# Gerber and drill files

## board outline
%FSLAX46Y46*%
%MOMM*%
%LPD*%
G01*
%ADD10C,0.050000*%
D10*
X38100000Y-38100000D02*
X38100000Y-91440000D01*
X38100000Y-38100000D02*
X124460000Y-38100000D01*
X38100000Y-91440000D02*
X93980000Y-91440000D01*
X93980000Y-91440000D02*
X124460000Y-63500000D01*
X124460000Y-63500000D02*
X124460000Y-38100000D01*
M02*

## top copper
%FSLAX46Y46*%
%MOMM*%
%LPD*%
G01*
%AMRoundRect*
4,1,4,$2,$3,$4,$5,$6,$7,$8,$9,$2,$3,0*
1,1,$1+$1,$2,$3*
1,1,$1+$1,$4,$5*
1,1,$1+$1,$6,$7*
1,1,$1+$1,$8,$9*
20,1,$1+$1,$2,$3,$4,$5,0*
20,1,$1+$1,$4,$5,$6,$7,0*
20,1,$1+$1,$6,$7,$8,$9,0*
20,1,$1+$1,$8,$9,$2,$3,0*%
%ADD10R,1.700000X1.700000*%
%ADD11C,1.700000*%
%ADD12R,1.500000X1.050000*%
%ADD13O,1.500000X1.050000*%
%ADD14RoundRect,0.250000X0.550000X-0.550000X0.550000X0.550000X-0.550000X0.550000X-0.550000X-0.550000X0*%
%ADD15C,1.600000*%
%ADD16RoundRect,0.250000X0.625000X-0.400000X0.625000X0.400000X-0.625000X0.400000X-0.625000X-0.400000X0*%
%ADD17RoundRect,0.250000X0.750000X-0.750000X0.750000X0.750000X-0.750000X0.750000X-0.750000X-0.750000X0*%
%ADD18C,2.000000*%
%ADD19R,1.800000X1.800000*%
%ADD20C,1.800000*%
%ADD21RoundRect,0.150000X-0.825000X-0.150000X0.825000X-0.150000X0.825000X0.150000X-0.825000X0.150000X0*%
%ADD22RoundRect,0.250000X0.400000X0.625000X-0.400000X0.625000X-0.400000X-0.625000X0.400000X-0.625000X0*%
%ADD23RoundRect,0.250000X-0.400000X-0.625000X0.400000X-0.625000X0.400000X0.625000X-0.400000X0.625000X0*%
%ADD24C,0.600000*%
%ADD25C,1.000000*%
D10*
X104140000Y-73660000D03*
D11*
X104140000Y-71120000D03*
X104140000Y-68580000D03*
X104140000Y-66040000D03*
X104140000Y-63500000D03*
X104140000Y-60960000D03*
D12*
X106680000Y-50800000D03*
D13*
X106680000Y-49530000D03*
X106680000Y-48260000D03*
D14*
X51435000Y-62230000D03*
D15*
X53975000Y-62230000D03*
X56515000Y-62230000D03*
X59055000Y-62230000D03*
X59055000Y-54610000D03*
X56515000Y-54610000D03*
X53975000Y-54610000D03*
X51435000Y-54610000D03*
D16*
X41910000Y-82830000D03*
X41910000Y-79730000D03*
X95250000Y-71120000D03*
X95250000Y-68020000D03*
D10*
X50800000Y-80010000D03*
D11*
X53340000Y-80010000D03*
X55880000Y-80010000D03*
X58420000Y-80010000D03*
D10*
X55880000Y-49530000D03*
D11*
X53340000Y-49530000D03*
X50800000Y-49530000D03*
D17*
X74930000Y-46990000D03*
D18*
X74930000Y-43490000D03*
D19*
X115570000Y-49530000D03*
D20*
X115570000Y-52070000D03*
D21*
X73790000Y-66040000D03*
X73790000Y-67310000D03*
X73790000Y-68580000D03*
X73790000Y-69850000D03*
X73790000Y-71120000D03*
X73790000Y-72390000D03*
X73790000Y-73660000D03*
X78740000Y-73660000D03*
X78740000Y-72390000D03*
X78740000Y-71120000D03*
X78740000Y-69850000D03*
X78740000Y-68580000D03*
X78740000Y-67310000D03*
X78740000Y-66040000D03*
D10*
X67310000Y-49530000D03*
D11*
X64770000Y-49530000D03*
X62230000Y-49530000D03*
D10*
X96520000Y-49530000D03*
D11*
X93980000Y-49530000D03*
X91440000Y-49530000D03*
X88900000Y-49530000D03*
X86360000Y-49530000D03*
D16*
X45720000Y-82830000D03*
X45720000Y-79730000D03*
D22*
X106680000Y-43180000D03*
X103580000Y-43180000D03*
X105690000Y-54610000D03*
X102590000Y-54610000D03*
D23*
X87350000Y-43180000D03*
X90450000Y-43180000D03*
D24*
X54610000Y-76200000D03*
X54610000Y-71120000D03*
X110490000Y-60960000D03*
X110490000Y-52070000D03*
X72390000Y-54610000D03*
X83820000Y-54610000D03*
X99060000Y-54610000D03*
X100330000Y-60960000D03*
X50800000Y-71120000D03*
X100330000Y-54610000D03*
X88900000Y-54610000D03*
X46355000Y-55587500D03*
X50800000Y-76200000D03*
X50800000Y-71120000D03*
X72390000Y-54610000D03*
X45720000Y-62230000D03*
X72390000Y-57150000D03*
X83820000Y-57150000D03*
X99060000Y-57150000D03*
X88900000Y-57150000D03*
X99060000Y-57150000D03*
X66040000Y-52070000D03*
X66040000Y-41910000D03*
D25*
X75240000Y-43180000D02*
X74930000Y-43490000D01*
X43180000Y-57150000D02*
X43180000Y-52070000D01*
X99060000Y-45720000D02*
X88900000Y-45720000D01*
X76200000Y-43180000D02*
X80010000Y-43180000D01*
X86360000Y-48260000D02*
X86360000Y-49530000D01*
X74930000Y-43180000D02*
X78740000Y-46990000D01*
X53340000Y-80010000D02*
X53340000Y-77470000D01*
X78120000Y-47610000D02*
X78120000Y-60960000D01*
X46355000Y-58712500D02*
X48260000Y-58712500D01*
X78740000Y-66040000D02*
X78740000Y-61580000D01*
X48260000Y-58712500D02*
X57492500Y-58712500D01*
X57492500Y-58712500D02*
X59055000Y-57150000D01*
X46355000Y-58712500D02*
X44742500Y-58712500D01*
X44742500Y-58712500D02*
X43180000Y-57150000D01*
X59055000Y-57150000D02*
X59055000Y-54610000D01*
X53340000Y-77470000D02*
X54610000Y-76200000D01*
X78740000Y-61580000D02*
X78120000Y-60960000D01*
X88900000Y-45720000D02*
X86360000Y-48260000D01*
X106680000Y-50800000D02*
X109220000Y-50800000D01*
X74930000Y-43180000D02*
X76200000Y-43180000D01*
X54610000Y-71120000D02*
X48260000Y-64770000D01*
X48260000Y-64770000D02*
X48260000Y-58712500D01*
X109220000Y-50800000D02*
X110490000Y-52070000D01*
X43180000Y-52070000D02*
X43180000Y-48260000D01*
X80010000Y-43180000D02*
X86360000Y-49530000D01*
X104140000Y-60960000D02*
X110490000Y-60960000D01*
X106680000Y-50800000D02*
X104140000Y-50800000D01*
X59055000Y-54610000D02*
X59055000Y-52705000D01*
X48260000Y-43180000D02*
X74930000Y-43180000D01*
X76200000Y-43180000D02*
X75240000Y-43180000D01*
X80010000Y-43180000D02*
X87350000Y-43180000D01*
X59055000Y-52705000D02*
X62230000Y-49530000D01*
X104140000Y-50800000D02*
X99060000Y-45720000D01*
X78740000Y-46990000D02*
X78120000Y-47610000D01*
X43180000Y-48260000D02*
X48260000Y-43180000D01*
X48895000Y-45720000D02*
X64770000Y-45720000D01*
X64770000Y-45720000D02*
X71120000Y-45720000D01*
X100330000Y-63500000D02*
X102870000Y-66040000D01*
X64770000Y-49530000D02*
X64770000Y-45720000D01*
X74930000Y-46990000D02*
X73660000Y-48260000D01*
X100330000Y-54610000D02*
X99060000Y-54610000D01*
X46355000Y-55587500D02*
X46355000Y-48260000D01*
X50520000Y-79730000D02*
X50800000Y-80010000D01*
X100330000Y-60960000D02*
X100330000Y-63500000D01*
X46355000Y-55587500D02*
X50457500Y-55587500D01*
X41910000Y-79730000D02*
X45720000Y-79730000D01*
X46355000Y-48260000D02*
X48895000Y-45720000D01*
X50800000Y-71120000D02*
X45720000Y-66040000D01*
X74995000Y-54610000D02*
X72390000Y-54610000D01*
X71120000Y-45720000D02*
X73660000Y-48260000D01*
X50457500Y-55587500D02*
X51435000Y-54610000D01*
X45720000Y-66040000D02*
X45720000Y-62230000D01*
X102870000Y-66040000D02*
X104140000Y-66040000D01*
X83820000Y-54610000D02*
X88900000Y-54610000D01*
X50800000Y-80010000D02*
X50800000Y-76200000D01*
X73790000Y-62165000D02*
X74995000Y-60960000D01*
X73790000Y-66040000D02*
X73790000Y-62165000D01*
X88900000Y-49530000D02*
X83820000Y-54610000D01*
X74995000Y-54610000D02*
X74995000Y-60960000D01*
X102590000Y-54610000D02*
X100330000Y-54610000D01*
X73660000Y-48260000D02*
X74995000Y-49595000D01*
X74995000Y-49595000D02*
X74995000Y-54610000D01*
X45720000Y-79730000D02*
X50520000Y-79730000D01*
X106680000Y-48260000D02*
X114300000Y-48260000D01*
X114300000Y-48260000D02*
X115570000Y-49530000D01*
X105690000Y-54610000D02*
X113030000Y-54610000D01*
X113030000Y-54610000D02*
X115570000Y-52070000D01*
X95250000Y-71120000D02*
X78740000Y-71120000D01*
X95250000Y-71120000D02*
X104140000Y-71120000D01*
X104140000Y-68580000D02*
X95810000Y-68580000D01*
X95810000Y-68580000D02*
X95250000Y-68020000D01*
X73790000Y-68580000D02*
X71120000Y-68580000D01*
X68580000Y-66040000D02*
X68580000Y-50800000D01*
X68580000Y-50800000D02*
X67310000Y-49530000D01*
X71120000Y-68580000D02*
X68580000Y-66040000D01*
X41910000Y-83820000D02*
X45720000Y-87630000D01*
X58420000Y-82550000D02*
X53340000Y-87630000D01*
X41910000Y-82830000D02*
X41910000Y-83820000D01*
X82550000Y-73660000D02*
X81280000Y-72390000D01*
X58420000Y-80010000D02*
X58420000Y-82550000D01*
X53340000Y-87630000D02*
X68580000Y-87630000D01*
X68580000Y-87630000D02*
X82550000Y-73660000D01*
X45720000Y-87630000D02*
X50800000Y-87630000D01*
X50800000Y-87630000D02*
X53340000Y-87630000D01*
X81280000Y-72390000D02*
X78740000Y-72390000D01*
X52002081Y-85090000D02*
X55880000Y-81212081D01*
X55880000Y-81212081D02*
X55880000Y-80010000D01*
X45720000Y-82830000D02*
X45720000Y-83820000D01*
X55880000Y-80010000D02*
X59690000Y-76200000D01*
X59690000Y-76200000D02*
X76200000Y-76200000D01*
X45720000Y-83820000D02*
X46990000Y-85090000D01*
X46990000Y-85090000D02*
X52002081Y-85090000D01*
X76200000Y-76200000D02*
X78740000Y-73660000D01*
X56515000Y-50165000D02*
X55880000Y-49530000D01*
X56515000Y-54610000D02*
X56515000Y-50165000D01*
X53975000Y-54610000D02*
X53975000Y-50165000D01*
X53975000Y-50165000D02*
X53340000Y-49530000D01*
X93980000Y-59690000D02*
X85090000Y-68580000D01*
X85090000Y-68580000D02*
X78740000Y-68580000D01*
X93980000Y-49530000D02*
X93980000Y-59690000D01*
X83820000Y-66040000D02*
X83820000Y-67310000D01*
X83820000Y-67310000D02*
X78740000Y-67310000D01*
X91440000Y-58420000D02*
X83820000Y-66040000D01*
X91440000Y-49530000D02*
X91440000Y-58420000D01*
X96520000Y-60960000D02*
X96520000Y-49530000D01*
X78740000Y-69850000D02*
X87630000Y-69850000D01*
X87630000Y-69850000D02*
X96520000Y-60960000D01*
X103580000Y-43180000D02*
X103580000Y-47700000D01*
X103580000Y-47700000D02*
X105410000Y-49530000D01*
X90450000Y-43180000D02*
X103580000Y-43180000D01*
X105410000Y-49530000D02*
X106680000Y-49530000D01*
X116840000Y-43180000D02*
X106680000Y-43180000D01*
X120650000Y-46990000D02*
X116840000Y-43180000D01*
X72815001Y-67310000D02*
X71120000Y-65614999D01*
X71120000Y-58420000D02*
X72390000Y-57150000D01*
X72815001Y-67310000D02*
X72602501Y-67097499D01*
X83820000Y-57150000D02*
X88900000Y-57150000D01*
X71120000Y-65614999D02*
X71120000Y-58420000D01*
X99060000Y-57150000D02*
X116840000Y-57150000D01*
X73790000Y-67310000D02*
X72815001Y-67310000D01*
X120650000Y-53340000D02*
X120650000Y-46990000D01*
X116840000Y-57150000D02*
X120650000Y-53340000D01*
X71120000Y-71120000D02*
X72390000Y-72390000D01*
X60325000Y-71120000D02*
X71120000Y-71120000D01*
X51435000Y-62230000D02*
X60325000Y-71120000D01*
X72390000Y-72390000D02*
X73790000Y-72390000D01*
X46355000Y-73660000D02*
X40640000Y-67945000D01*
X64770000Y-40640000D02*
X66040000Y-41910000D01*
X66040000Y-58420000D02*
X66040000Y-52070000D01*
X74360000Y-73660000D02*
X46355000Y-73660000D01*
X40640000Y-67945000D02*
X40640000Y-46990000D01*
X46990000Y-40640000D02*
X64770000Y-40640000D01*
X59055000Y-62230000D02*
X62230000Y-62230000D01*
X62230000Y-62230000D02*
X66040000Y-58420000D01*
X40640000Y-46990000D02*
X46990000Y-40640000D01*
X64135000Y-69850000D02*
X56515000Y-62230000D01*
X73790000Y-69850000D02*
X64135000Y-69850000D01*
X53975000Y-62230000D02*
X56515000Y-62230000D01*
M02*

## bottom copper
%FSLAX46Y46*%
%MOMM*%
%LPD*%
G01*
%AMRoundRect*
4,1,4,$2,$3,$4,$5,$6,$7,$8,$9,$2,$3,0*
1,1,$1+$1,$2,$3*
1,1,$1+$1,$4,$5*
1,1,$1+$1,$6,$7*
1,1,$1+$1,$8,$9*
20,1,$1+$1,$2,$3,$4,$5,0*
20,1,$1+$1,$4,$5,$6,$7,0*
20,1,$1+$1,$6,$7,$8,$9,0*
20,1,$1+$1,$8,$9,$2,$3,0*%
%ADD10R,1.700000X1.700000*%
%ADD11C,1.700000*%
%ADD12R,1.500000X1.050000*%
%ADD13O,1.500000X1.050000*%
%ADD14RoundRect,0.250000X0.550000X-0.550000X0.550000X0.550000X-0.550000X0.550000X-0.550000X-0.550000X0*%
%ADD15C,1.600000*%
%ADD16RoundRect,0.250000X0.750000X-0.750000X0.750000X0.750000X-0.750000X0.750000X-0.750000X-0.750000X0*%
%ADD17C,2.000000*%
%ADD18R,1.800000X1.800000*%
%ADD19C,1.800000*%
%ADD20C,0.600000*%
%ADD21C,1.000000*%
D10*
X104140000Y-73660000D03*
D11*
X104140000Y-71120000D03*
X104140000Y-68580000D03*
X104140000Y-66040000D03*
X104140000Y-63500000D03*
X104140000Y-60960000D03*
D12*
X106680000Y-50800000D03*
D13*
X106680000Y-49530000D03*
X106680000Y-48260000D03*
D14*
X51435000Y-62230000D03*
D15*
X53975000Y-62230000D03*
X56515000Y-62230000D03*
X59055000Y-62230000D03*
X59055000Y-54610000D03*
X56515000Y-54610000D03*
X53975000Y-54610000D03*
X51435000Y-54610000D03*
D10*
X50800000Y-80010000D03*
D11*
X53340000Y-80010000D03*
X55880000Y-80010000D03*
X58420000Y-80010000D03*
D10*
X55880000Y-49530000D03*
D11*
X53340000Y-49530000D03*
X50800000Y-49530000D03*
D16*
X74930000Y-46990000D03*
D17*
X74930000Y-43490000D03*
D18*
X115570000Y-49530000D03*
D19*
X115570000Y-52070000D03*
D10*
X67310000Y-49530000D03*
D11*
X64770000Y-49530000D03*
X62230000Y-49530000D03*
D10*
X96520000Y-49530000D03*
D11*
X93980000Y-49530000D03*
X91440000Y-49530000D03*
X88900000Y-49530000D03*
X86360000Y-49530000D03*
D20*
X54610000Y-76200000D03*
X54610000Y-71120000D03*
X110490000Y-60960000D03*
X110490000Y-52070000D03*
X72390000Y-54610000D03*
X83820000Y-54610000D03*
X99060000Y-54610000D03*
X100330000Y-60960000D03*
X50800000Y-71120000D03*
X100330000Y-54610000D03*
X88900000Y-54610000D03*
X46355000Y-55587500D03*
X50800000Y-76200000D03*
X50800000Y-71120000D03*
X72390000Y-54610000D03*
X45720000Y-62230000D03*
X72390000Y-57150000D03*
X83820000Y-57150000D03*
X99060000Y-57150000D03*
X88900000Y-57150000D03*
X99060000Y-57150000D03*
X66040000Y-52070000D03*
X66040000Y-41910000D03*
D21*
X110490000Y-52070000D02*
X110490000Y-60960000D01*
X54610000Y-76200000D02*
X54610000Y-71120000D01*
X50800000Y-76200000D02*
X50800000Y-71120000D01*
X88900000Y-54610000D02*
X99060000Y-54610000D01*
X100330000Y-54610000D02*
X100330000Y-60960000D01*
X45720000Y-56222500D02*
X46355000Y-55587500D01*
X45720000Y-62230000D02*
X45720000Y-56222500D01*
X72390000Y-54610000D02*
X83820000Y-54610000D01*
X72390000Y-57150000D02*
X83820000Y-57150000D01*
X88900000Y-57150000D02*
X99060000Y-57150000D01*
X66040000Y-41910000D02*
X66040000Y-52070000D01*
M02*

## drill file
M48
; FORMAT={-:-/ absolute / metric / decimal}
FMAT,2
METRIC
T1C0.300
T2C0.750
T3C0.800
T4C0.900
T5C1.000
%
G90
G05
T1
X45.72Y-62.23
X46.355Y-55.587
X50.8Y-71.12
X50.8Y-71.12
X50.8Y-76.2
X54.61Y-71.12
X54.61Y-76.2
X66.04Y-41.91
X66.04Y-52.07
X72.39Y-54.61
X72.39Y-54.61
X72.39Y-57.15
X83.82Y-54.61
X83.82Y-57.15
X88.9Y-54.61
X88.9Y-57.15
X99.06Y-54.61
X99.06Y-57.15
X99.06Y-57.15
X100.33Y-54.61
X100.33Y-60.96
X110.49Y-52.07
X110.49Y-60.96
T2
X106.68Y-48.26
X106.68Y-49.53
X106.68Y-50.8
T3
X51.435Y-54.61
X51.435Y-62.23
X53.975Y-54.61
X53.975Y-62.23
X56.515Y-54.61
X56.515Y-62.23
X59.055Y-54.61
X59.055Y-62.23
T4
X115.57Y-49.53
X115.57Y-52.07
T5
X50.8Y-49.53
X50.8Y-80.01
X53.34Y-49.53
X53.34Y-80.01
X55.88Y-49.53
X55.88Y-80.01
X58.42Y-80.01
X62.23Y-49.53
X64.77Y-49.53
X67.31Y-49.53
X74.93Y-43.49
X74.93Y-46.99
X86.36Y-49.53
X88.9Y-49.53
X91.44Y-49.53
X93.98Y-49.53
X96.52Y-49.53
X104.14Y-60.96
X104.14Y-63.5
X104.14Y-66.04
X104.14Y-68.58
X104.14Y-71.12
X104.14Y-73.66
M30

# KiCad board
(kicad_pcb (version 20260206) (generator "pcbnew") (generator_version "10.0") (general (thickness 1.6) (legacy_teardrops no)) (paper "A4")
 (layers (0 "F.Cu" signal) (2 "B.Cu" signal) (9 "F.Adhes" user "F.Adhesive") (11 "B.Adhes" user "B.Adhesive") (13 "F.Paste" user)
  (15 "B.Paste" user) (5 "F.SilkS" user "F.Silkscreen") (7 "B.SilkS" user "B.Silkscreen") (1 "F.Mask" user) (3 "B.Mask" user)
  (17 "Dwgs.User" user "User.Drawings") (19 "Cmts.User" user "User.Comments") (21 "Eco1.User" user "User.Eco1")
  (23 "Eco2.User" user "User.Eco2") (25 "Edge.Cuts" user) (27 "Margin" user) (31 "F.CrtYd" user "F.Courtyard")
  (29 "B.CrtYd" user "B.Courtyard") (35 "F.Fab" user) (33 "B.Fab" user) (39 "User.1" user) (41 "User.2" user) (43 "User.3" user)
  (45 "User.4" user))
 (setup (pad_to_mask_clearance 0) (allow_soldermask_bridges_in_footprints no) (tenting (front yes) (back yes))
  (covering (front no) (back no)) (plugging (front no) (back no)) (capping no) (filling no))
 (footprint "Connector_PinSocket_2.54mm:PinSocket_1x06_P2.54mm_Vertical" (layer "F.Cu") (at 104.14 73.66 180)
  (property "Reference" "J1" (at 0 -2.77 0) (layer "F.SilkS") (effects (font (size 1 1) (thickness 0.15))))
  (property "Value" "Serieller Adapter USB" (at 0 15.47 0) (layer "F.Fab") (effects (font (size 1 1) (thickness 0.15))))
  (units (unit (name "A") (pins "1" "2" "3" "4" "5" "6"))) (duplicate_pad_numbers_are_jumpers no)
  (pad "1" thru_hole rect (at 0 0 180) (size 1.7 1.7) (drill 1) (layers "*.Cu" "*.Mask") (remove_unused_layers no)
   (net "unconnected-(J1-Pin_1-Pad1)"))
  (pad "2" thru_hole circle (at 0 2.54 180) (size 1.7 1.7) (drill 1) (layers "*.Cu" "*.Mask") (remove_unused_layers no)
   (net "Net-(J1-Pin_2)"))
  (pad "3" thru_hole circle (at 0 5.08 180) (size 1.7 1.7) (drill 1) (layers "*.Cu" "*.Mask") (remove_unused_layers no)
   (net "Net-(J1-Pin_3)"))
  (pad "4" thru_hole circle (at 0 7.62 180) (size 1.7 1.7) (drill 1) (layers "*.Cu" "*.Mask") (remove_unused_layers no) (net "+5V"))
  (pad "5" thru_hole circle (at 0 10.16 180) (size 1.7 1.7) (drill 1) (layers "*.Cu" "*.Mask") (remove_unused_layers no)
   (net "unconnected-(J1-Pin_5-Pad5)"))
  (pad "6" thru_hole circle (at 0 12.7 180) (size 1.7 1.7) (drill 1) (layers "*.Cu" "*.Mask") (remove_unused_layers no) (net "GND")))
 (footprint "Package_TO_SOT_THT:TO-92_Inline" (layer "F.Cu") (at 106.68 50.8 90)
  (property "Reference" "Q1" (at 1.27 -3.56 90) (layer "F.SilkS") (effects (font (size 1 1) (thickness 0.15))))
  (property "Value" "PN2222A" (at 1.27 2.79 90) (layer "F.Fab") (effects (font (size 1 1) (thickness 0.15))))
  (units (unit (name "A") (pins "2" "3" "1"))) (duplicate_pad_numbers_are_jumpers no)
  (pad "1" thru_hole rect (at 0 0 90) (size 1.05 1.5) (drill 0.75) (layers "*.Cu" "*.Mask") (remove_unused_layers no) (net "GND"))
  (pad "2" thru_hole oval (at 1.27 0 90) (size 1.05 1.5) (drill 0.75) (layers "*.Cu" "*.Mask") (remove_unused_layers no) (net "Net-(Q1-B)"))
  (pad "3" thru_hole oval (at 2.54 0 90) (size 1.05 1.5) (drill 0.75) (layers "*.Cu" "*.Mask") (remove_unused_layers no) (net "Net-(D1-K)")))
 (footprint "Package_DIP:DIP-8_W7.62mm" (layer "F.Cu") (at 51.435 62.23 90)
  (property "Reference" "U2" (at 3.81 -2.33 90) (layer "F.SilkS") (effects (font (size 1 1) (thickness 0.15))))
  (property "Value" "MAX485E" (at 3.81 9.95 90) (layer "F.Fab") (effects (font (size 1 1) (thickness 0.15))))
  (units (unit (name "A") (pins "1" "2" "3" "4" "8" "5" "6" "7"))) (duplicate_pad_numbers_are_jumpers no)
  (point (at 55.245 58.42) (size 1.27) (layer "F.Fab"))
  (pad "1" thru_hole roundrect (at 0 0 90) (size 1.6 1.6) (drill 0.8) (layers "*.Cu" "*.Mask") (remove_unused_layers no)
   (roundrect_rratio 0.15625) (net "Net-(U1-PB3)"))
  (pad "2" thru_hole circle (at 0 2.54 90) (size 1.6 1.6) (drill 0.8) (layers "*.Cu" "*.Mask") (remove_unused_layers no)
   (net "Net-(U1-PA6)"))
  (pad "3" thru_hole circle (at 0 5.08 90) (size 1.6 1.6) (drill 0.8) (layers "*.Cu" "*.Mask") (remove_unused_layers no)
   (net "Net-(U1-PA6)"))
  (pad "4" thru_hole circle (at 0 7.62 90) (size 1.6 1.6) (drill 0.8) (layers "*.Cu" "*.Mask") (remove_unused_layers no)
   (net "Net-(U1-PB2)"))
  (pad "5" thru_hole circle (at 7.62 7.62 90) (size 1.6 1.6) (drill 0.8) (layers "*.Cu" "*.Mask") (remove_unused_layers no) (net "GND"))
  (pad "6" thru_hole circle (at 7.62 5.08 90) (size 1.6 1.6) (drill 0.8) (layers "*.Cu" "*.Mask") (remove_unused_layers no)
   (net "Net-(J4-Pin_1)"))
  (pad "7" thru_hole circle (at 7.62 2.54 90) (size 1.6 1.6) (drill 0.8) (layers "*.Cu" "*.Mask") (remove_unused_layers no)
   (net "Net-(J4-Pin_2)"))
  (pad "8" thru_hole circle (at 7.62 0 90) (size 1.6 1.6) (drill 0.8) (layers "*.Cu" "*.Mask") (remove_unused_layers no) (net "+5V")))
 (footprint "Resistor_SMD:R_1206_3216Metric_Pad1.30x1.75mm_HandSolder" (layer "F.Cu") (at 41.91 81.28 90)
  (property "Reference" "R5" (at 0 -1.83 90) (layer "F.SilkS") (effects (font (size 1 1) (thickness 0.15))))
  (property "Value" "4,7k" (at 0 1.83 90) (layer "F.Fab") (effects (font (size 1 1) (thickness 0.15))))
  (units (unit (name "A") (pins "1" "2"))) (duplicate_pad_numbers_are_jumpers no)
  (pad "1" smd roundrect (at -1.55 0 90) (size 1.3 1.75) (layers "F.Cu" "F.Mask" "F.Paste") (roundrect_rratio 0.192308)
   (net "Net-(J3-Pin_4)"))
  (pad "2" smd roundrect (at 1.55 0 90) (size 1.3 1.75) (layers "F.Cu" "F.Mask" "F.Paste") (roundrect_rratio 0.192308) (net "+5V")))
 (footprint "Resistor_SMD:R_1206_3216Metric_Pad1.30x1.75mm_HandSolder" (layer "F.Cu") (at 95.25 69.57 90)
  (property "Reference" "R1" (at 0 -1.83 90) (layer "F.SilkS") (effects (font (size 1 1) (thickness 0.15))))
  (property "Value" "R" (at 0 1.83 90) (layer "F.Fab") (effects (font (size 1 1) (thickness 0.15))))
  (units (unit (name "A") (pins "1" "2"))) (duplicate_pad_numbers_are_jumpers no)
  (pad "1" smd roundrect (at -1.55 0 90) (size 1.3 1.75) (layers "F.Cu" "F.Mask" "F.Paste") (roundrect_rratio 0.192308)
   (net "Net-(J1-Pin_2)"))
  (pad "2" smd roundrect (at 1.55 0 90) (size 1.3 1.75) (layers "F.Cu" "F.Mask" "F.Paste") (roundrect_rratio 0.192308)
   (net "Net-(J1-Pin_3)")))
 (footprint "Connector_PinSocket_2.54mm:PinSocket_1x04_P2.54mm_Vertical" (layer "F.Cu") (at 50.8 80.01 90)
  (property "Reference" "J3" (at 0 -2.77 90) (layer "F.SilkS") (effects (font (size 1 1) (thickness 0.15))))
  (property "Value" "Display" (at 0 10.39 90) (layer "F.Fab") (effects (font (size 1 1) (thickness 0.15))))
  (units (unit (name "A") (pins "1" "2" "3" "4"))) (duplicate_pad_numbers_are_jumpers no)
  (pad "1" thru_hole rect (at 0 0 90) (size 1.7 1.7) (drill 1) (layers "*.Cu" "*.Mask") (remove_unused_layers no) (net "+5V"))
  (pad "2" thru_hole circle (at 0 2.54 90) (size 1.7 1.7) (drill 1) (layers "*.Cu" "*.Mask") (remove_unused_layers no) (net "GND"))
  (pad "3" thru_hole circle (at 0 5.08 90) (size 1.7 1.7) (drill 1) (layers "*.Cu" "*.Mask") (remove_unused_layers no)
   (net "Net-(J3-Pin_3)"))
  (pad "4" thru_hole circle (at 0 7.62 90) (size 1.7 1.7) (drill 1) (layers "*.Cu" "*.Mask") (remove_unused_layers no)
   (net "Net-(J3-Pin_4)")))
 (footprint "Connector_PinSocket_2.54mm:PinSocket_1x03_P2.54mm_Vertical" (layer "F.Cu") (at 55.88 49.53 -90)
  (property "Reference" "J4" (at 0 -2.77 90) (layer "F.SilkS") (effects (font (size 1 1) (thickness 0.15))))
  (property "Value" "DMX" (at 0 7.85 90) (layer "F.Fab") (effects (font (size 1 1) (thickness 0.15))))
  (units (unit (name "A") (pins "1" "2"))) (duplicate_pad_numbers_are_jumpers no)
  (pad "1" thru_hole rect (at 0 0 270) (size 1.7 1.7) (drill 1) (layers "*.Cu" "*.Mask") (remove_unused_layers no) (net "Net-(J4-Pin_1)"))
  (pad "2" thru_hole circle (at 0 2.54 270) (size 1.7 1.7) (drill 1) (layers "*.Cu" "*.Mask") (remove_unused_layers no)
   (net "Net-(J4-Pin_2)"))
  (pad "3" thru_hole circle (at 0 5.08 270) (size 1.7 1.7) (drill 1) (layers "*.Cu" "*.Mask") (remove_unused_layers no)))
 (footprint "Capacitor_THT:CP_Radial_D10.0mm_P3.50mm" (layer "F.Cu") (at 74.93 46.99 90)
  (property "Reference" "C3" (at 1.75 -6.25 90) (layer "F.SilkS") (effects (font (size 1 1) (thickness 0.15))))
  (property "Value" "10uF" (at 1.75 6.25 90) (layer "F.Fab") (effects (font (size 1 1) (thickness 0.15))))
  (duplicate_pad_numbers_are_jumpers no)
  (pad "1" thru_hole roundrect (at 0 0 90) (size 2 2) (drill 1) (layers "*.Cu" "*.Mask") (remove_unused_layers no) (roundrect_rratio 0.125)
   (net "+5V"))
  (pad "2" thru_hole circle (at 3.5 0 90) (size 2 2) (drill 1) (layers "*.Cu" "*.Mask") (remove_unused_layers no) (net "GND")))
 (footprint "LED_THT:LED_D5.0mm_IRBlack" (layer "F.Cu") (at 115.57 49.53 -90)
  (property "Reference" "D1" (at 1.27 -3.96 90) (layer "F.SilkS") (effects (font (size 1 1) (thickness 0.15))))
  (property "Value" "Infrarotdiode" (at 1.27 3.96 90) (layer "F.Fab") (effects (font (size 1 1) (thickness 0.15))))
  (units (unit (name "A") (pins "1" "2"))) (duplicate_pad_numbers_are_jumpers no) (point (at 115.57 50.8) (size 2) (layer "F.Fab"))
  (pad "1" thru_hole rect (at 0 0 270) (size 1.8 1.8) (drill 0.9) (layers "*.Cu" "*.Mask") (remove_unused_layers no) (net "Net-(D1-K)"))
  (pad "2" thru_hole circle (at 2.54 0 270) (size 1.8 1.8) (drill 0.9) (layers "*.Cu" "*.Mask") (remove_unused_layers no) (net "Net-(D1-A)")))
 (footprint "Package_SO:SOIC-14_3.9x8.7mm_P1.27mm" (layer "F.Cu") (at 76.265 69.85)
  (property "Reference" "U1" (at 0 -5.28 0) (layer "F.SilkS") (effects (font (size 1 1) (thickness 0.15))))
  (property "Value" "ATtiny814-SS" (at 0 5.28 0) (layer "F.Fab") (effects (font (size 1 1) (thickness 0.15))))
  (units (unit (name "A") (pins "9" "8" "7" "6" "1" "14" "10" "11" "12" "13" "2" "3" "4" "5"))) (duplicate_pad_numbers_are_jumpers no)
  (pad "1" smd roundrect (at -2.475 -3.81) (size 1.95 0.6) (layers "F.Cu" "F.Mask" "F.Paste") (roundrect_rratio 0.25) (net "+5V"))
  (pad "2" smd roundrect (at -2.475 -2.54) (size 1.95 0.6) (layers "F.Cu" "F.Mask" "F.Paste") (roundrect_rratio 0.25) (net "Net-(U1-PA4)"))
  (pad "3" smd roundrect (at -2.475 -1.27) (size 1.95 0.6) (layers "F.Cu" "F.Mask" "F.Paste") (roundrect_rratio 0.25) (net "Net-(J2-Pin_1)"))
  (pad "4" smd roundrect (at -2.475 0) (size 1.95 0.6) (layers "F.Cu" "F.Mask" "F.Paste") (roundrect_rratio 0.25) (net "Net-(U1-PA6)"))
  (pad "5" smd roundrect (at -2.475 1.27) (size 1.95 0.6) (layers "F.Cu" "F.Mask" "F.Paste") (roundrect_rratio 0.25)
   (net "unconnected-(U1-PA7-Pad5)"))
  (pad "6" smd roundrect (at -2.475 2.54) (size 1.95 0.6) (layers "F.Cu" "F.Mask" "F.Paste") (roundrect_rratio 0.25) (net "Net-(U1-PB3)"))
  (pad "7" smd roundrect (at -2.475 3.81) (size 1.95 0.6) (layers "F.Cu" "F.Mask" "F.Paste") (roundrect_rratio 0.25) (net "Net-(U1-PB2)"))
  (pad "8" smd roundrect (at 2.475 3.81) (size 1.95 0.6) (layers "F.Cu" "F.Mask" "F.Paste") (roundrect_rratio 0.25) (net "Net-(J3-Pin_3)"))
  (pad "9" smd roundrect (at 2.475 2.54) (size 1.95 0.6) (layers "F.Cu" "F.Mask" "F.Paste") (roundrect_rratio 0.25) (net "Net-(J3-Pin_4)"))
  (pad "10" smd roundrect (at 2.475 1.27) (size 1.95 0.6) (layers "F.Cu" "F.Mask" "F.Paste") (roundrect_rratio 0.25) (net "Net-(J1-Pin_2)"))
  (pad "11" smd roundrect (at 2.475 0) (size 1.95 0.6) (layers "F.Cu" "F.Mask" "F.Paste") (roundrect_rratio 0.25) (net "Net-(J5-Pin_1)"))
  (pad "12" smd roundrect (at 2.475 -1.27) (size 1.95 0.6) (layers "F.Cu" "F.Mask" "F.Paste") (roundrect_rratio 0.25) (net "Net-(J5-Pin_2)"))
  (pad "13" smd roundrect (at 2.475 -2.54) (size 1.95 0.6) (layers "F.Cu" "F.Mask" "F.Paste") (roundrect_rratio 0.25) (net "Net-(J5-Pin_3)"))
  (pad "14" smd roundrect (at 2.475 -3.81) (size 1.95 0.6) (layers "F.Cu" "F.Mask" "F.Paste") (roundrect_rratio 0.25) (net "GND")))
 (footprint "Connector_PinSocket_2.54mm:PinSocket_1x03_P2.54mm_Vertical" (layer "F.Cu") (at 67.31 49.53 -90)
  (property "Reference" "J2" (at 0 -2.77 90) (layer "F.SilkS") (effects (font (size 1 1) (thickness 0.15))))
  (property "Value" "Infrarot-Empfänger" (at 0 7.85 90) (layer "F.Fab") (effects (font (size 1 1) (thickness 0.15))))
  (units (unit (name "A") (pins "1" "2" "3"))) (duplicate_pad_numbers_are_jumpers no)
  (pad "1" thru_hole rect (at 0 0 270) (size 1.7 1.7) (drill 1) (layers "*.Cu" "*.Mask") (remove_unused_layers no) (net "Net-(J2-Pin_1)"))
  (pad "2" thru_hole circle (at 0 2.54 270) (size 1.7 1.7) (drill 1) (layers "*.Cu" "*.Mask") (remove_unused_layers no) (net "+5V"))
  (pad "3" thru_hole circle (at 0 5.08 270) (size 1.7 1.7) (drill 1) (layers "*.Cu" "*.Mask") (remove_unused_layers no) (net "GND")))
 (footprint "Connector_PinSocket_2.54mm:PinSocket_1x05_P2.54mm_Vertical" (layer "F.Cu") (at 96.52 49.53 -90)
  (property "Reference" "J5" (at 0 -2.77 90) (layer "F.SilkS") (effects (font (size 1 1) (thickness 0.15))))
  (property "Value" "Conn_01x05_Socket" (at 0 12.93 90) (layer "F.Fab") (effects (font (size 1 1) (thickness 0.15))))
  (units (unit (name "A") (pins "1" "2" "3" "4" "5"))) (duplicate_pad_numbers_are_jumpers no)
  (pad "1" thru_hole rect (at 0 0 270) (size 1.7 1.7) (drill 1) (layers "*.Cu" "*.Mask") (remove_unused_layers no) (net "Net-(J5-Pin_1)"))
  (pad "2" thru_hole circle (at 0 2.54 270) (size 1.7 1.7) (drill 1) (layers "*.Cu" "*.Mask") (remove_unused_layers no)
   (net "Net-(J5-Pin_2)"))
  (pad "3" thru_hole circle (at 0 5.08 270) (size 1.7 1.7) (drill 1) (layers "*.Cu" "*.Mask") (remove_unused_layers no)
   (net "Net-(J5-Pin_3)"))
  (pad "4" thru_hole circle (at 0 7.62 270) (size 1.7 1.7) (drill 1) (layers "*.Cu" "*.Mask") (remove_unused_layers no) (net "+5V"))
  (pad "5" thru_hole circle (at 0 10.16 270) (size 1.7 1.7) (drill 1) (layers "*.Cu" "*.Mask") (remove_unused_layers no) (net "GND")))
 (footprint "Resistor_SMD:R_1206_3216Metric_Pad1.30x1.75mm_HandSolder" (layer "F.Cu") (at 45.72 81.28 90)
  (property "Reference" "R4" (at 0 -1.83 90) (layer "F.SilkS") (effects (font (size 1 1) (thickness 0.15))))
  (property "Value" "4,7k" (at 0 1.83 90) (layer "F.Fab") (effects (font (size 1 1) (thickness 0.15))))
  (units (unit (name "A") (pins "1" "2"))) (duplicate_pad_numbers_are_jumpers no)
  (pad "1" smd roundrect (at -1.55 0 90) (size 1.3 1.75) (layers "F.Cu" "F.Mask" "F.Paste") (roundrect_rratio 0.192308)
   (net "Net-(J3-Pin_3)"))
  (pad "2" smd roundrect (at 1.55 0 90) (size 1.3 1.75) (layers "F.Cu" "F.Mask" "F.Paste") (roundrect_rratio 0.192308) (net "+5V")))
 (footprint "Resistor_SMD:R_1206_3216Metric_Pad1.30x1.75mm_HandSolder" (layer "F.Cu") (at 105.13 43.18 180)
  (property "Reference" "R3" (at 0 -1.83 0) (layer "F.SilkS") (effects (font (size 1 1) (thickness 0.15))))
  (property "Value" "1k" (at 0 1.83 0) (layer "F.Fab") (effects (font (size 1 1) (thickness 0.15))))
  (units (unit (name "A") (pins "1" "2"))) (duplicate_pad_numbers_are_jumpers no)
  (pad "1" smd roundrect (at -1.55 0 180) (size 1.3 1.75) (layers "F.Cu" "F.Mask" "F.Paste") (roundrect_rratio 0.192308)
   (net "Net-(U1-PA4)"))
  (pad "2" smd roundrect (at 1.55 0 180) (size 1.3 1.75) (layers "F.Cu" "F.Mask" "F.Paste") (roundrect_rratio 0.192308) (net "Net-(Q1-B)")))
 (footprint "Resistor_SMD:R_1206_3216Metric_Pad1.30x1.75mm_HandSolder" (layer "F.Cu") (at 104.14 54.61 180)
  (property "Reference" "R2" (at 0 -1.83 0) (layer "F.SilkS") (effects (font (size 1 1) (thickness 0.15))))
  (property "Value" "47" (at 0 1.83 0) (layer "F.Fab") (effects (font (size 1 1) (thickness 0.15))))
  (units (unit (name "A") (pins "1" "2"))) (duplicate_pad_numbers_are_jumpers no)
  (pad "1" smd roundrect (at -1.55 0 180) (size 1.3 1.75) (layers "F.Cu" "F.Mask" "F.Paste") (roundrect_rratio 0.192308) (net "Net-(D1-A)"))
  (pad "2" smd roundrect (at 1.55 0 180) (size 1.3 1.75) (layers "F.Cu" "F.Mask" "F.Paste") (roundrect_rratio 0.192308) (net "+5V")))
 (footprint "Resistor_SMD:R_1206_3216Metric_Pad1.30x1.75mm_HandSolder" (layer "F.Cu") (at 88.9 43.18)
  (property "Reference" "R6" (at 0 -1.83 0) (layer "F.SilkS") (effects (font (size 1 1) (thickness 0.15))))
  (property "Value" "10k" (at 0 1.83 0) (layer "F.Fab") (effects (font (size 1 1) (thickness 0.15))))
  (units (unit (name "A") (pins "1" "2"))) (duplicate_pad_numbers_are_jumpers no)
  (pad "1" smd roundrect (at -1.55 0) (size 1.3 1.75) (layers "F.Cu" "F.Mask" "F.Paste") (roundrect_rratio 0.192308) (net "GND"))
  (pad "2" smd roundrect (at 1.55 0) (size 1.3 1.75) (layers "F.Cu" "F.Mask" "F.Paste") (roundrect_rratio 0.192308) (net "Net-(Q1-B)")))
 (gr_line (start 38.1 38.1) (end 38.1 91.44) (stroke (width 0.05) (type default)) (layer "Edge.Cuts"))
 (gr_line (start 38.1 38.1) (end 124.46 38.1) (stroke (width 0.05) (type default)) (layer "Edge.Cuts"))
 (gr_line (start 38.1 91.44) (end 93.98 91.44) (stroke (width 0.05) (type default)) (layer "Edge.Cuts"))
 (gr_line (start 93.98 91.44) (end 124.46 63.5) (stroke (width 0.05) (type default)) (layer "Edge.Cuts"))
 (gr_line (start 124.46 63.5) (end 124.46 38.1) (stroke (width 0.05) (type default)) (layer "Edge.Cuts"))
 (segment (start 75.24 43.18) (end 74.93 43.49) (width 1) (layer "F.Cu") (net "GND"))
 (segment (start 43.18 57.15) (end 43.18 52.07) (width 1) (layer "F.Cu") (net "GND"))
 (segment (start 99.06 45.72) (end 88.9 45.72) (width 1) (layer "F.Cu") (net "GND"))
 (segment (start 76.2 43.18) (end 80.01 43.18) (width 1) (layer "F.Cu") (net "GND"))
 (segment (start 86.36 48.26) (end 86.36 49.53) (width 1) (layer "F.Cu") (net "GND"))
 (segment (start 74.93 43.18) (end 78.74 46.99) (width 1) (layer "F.Cu") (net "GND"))
 (segment (start 53.34 80.01) (end 53.34 77.47) (width 1) (layer "F.Cu") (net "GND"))
 (segment (start 78.12 47.61) (end 78.12 60.96) (width 1) (layer "F.Cu") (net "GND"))
 (segment (start 46.355 58.7125) (end 48.26 58.7125) (width 1) (layer "F.Cu") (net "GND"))
 (segment (start 78.74 66.04) (end 78.74 61.58) (width 1) (layer "F.Cu") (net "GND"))
 (segment (start 48.26 58.7125) (end 57.4925 58.7125) (width 1) (layer "F.Cu") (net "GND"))
 (segment (start 57.4925 58.7125) (end 59.055 57.15) (width 1) (layer "F.Cu") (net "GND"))
 (segment (start 46.355 58.7125) (end 44.7425 58.7125) (width 1) (layer "F.Cu") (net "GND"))
 (segment (start 44.7425 58.7125) (end 43.18 57.15) (width 1) (layer "F.Cu") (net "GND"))
 (segment (start 59.055 57.15) (end 59.055 54.61) (width 1) (layer "F.Cu") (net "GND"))
 (segment (start 53.34 77.47) (end 54.61 76.2) (width 1) (layer "F.Cu") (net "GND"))
 (segment (start 78.74 61.58) (end 78.12 60.96) (width 1) (layer "F.Cu") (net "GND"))
 (segment (start 88.9 45.72) (end 86.36 48.26) (width 1) (layer "F.Cu") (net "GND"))
 (segment (start 106.68 50.8) (end 109.22 50.8) (width 1) (layer "F.Cu") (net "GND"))
 (segment (start 74.93 43.18) (end 76.2 43.18) (width 1) (layer "F.Cu") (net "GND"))
 (segment (start 54.61 71.12) (end 48.26 64.77) (width 1) (layer "F.Cu") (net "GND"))
 (segment (start 48.26 64.77) (end 48.26 58.7125) (width 1) (layer "F.Cu") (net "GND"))
 (segment (start 109.22 50.8) (end 110.49 52.07) (width 1) (layer "F.Cu") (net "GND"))
 (segment (start 43.18 52.07) (end 43.18 48.26) (width 1) (layer "F.Cu") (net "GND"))
 (segment (start 80.01 43.18) (end 86.36 49.53) (width 1) (layer "F.Cu") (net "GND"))
 (segment (start 104.14 60.96) (end 110.49 60.96) (width 1) (layer "F.Cu") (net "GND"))
 (segment (start 106.68 50.8) (end 104.14 50.8) (width 1) (layer "F.Cu") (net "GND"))
 (segment (start 59.055 54.61) (end 59.055 52.705) (width 1) (layer "F.Cu") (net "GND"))
 (segment (start 48.26 43.18) (end 74.93 43.18) (width 1) (layer "F.Cu") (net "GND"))
 (segment (start 76.2 43.18) (end 75.24 43.18) (width 1) (layer "F.Cu") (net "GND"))
 (segment (start 80.01 43.18) (end 87.35 43.18) (width 1) (layer "F.Cu") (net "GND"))
 (segment (start 59.055 52.705) (end 62.23 49.53) (width 1) (layer "F.Cu") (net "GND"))
 (segment (start 104.14 50.8) (end 99.06 45.72) (width 1) (layer "F.Cu") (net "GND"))
 (segment (start 78.74 46.99) (end 78.12 47.61) (width 1) (layer "F.Cu") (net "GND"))
 (segment (start 43.18 48.26) (end 48.26 43.18) (width 1) (layer "F.Cu") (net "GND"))
 (via (at 54.61 76.2) (size 0.6) (drill 0.3) (layers "F.Cu" "B.Cu") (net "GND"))
 (via (at 54.61 71.12) (size 0.6) (drill 0.3) (layers "F.Cu" "B.Cu") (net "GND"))
 (via (at 110.49 60.96) (size 0.6) (drill 0.3) (layers "F.Cu" "B.Cu") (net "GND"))
 (via (at 110.49 52.07) (size 0.6) (drill 0.3) (layers "F.Cu" "B.Cu") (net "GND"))
 (segment (start 110.49 52.07) (end 110.49 60.96) (width 1) (layer "B.Cu") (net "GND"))
 (segment (start 54.61 76.2) (end 54.61 71.12) (width 1) (layer "B.Cu") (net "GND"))
 (segment (start 48.895 45.72) (end 64.77 45.72) (width 1) (layer "F.Cu") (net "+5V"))
 (segment (start 64.77 45.72) (end 71.12 45.72) (width 1) (layer "F.Cu") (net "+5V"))
 (segment (start 100.33 63.5) (end 102.87 66.04) (width 1) (layer "F.Cu") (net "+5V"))
 (segment (start 64.77 49.53) (end 64.77 45.72) (width 1) (layer "F.Cu") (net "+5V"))
 (segment (start 74.93 46.99) (end 73.66 48.26) (width 1) (layer "F.Cu") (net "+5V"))
 (segment (start 100.33 54.61) (end 99.06 54.61) (width 1) (layer "F.Cu") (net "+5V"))
 (segment (start 46.355 55.5875) (end 46.355 48.26) (width 1) (layer "F.Cu") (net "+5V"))
 (segment (start 50.52 79.73) (end 50.8 80.01) (width 1) (layer "F.Cu") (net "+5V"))
 (segment (start 100.33 60.96) (end 100.33 63.5) (width 1) (layer "F.Cu") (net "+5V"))
 (segment (start 46.355 55.5875) (end 50.4575 55.5875) (width 1) (layer "F.Cu") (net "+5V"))
 (segment (start 41.91 79.73) (end 45.72 79.73) (width 1) (layer "F.Cu") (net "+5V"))
 (segment (start 46.355 48.26) (end 48.895 45.72) (width 1) (layer "F.Cu") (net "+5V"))
 (segment (start 50.8 71.12) (end 45.72 66.04) (width 1) (layer "F.Cu") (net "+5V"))
 (segment (start 74.995 54.61) (end 72.39 54.61) (width 1) (layer "F.Cu") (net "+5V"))
 (segment (start 71.12 45.72) (end 73.66 48.26) (width 1) (layer "F.Cu") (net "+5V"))
 (segment (start 50.4575 55.5875) (end 51.435 54.61) (width 1) (layer "F.Cu") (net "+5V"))
 (segment (start 45.72 66.04) (end 45.72 62.23) (width 1) (layer "F.Cu") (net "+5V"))
 (segment (start 102.87 66.04) (end 104.14 66.04) (width 1) (layer "F.Cu") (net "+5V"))
 (segment (start 83.82 54.61) (end 88.9 54.61) (width 1) (layer "F.Cu") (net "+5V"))
 (segment (start 50.8 80.01) (end 50.8 76.2) (width 1) (layer "F.Cu") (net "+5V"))
 (segment (start 73.79 62.165) (end 74.995 60.96) (width 1) (layer "F.Cu") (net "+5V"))
 (segment (start 73.79 66.04) (end 73.79 62.165) (width 1) (layer "F.Cu") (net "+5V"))
 (segment (start 88.9 49.53) (end 83.82 54.61) (width 1) (layer "F.Cu") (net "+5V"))
 (segment (start 74.995 54.61) (end 74.995 60.96) (width 1) (layer "F.Cu") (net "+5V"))
 (segment (start 102.59 54.61) (end 100.33 54.61) (width 1) (layer "F.Cu") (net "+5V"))
 (segment (start 73.66 48.26) (end 74.995 49.595) (width 1) (layer "F.Cu") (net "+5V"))
 (segment (start 74.995 49.595) (end 74.995 54.61) (width 1) (layer "F.Cu") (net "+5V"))
 (segment (start 45.72 79.73) (end 50.52 79.73) (width 1) (layer "F.Cu") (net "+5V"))
 (via (at 72.39 54.61) (size 0.6) (drill 0.3) (layers "F.Cu" "B.Cu") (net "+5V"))
 (via (at 83.82 54.61) (size 0.6) (drill 0.3) (layers "F.Cu" "B.Cu") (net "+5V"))
 (via (at 99.06 54.61) (size 0.6) (drill 0.3) (layers "F.Cu" "B.Cu") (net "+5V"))
 (via (at 100.33 60.96) (size 0.6) (drill 0.3) (layers "F.Cu" "B.Cu") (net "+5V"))
 (via (at 50.8 71.12) (size 0.6) (drill 0.3) (layers "F.Cu" "B.Cu") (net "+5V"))
 (via (at 100.33 54.61) (size 0.6) (drill 0.3) (layers "F.Cu" "B.Cu") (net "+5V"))
 (via (at 88.9 54.61) (size 0.6) (drill 0.3) (layers "F.Cu" "B.Cu") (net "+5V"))
 (via (at 46.355 55.5875) (size 0.6) (drill 0.3) (layers "F.Cu" "B.Cu") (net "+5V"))
 (via (at 50.8 76.2) (size 0.6) (drill 0.3) (layers "F.Cu" "B.Cu") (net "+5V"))
 (via (at 50.8 71.12) (size 0.6) (drill 0.3) (layers "F.Cu" "B.Cu") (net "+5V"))
 (via (at 72.39 54.61) (size 0.6) (drill 0.3) (layers "F.Cu" "B.Cu") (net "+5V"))
 (via (at 45.72 62.23) (size 0.6) (drill 0.3) (layers "F.Cu" "B.Cu") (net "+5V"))
 (segment (start 50.8 76.2) (end 50.8 71.12) (width 1) (layer "B.Cu") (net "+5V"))
 (segment (start 88.9 54.61) (end 99.06 54.61) (width 1) (layer "B.Cu") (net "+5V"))
 (segment (start 100.33 54.61) (end 100.33 60.96) (width 1) (layer "B.Cu") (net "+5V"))
 (segment (start 45.72 56.2225) (end 46.355 55.5875) (width 1) (layer "B.Cu") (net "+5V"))
 (segment (start 45.72 62.23) (end 45.72 56.2225) (width 1) (layer "B.Cu") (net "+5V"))
 (segment (start 72.39 54.61) (end 83.82 54.61) (width 1) (layer "B.Cu") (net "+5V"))
 (segment (start 106.68 48.26) (end 114.3 48.26) (width 1) (layer "F.Cu") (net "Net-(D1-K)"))
 (segment (start 114.3 48.26) (end 115.57 49.53) (width 1) (layer "F.Cu") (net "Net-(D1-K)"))
 (segment (start 105.69 54.61) (end 113.03 54.61) (width 1) (layer "F.Cu") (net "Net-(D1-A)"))
 (segment (start 113.03 54.61) (end 115.57 52.07) (width 1) (layer "F.Cu") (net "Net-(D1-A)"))
 (segment (start 95.25 71.12) (end 78.74 71.12) (width 1) (layer "F.Cu") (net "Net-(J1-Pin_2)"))
 (segment (start 95.25 71.12) (end 104.14 71.12) (width 1) (layer "F.Cu") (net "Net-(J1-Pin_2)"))
 (segment (start 104.14 68.58) (end 95.81 68.58) (width 1) (layer "F.Cu") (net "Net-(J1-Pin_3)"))
 (segment (start 95.81 68.58) (end 95.25 68.02) (width 1) (layer "F.Cu") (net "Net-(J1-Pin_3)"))
 (segment (start 73.79 68.58) (end 71.12 68.58) (width 1) (layer "F.Cu") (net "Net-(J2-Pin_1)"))
 (segment (start 68.58 66.04) (end 68.58 50.8) (width 1) (layer "F.Cu") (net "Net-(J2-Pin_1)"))
 (segment (start 68.58 50.8) (end 67.31 49.53) (width 1) (layer "F.Cu") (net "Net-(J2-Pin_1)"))
 (segment (start 71.12 68.58) (end 68.58 66.04) (width 1) (layer "F.Cu") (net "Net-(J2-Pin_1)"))
 (segment (start 41.91 83.82) (end 45.72 87.63) (width 1) (layer "F.Cu") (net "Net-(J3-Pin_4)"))
 (segment (start 58.42 82.55) (end 53.34 87.63) (width 1) (layer "F.Cu") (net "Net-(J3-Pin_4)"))
 (segment (start 41.91 82.83) (end 41.91 83.82) (width 1) (layer "F.Cu") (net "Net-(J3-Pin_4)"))
 (segment (start 82.55 73.66) (end 81.28 72.39) (width 1) (layer "F.Cu") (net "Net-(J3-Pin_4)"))
 (segment (start 58.42 80.01) (end 58.42 82.55) (width 1) (layer "F.Cu") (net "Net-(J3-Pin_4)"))
 (segment (start 53.34 87.63) (end 68.58 87.63) (width 1) (layer "F.Cu") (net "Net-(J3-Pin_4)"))
 (segment (start 68.58 87.63) (end 82.55 73.66) (width 1) (layer "F.Cu") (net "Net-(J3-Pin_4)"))
 (segment (start 45.72 87.63) (end 50.8 87.63) (width 1) (layer "F.Cu") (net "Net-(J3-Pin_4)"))
 (segment (start 50.8 87.63) (end 53.34 87.63) (width 1) (layer "F.Cu") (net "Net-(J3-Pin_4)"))
 (segment (start 81.28 72.39) (end 78.74 72.39) (width 1) (layer "F.Cu") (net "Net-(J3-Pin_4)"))
 (segment (start 52.002081 85.09) (end 55.88 81.212081) (width 1) (layer "F.Cu") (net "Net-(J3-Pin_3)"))
 (segment (start 55.88 81.212081) (end 55.88 80.01) (width 1) (layer "F.Cu") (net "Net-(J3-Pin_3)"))
 (segment (start 45.72 82.83) (end 45.72 83.82) (width 1) (layer "F.Cu") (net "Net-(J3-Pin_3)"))
 (segment (start 55.88 80.01) (end 59.69 76.2) (width 1) (layer "F.Cu") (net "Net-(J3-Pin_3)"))
 (segment (start 59.69 76.2) (end 76.2 76.2) (width 1) (layer "F.Cu") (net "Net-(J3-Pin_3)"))
 (segment (start 45.72 83.82) (end 46.99 85.09) (width 1) (layer "F.Cu") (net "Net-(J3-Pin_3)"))
 (segment (start 46.99 85.09) (end 52.002081 85.09) (width 1) (layer "F.Cu") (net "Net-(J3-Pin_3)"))
 (segment (start 76.2 76.2) (end 78.74 73.66) (width 1) (layer "F.Cu") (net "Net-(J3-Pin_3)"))
 (segment (start 56.515 50.165) (end 55.88 49.53) (width 1) (layer "F.Cu") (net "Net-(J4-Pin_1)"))
 (segment (start 56.515 54.61) (end 56.515 50.165) (width 1) (layer "F.Cu") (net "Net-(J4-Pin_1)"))
 (segment (start 53.975 54.61) (end 53.975 50.165) (width 1) (layer "F.Cu") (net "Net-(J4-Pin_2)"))
 (segment (start 53.975 50.165) (end 53.34 49.53) (width 1) (layer "F.Cu") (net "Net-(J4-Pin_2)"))
 (segment (start 93.98 59.69) (end 85.09 68.58) (width 1) (layer "F.Cu") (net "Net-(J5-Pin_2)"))
 (segment (start 85.09 68.58) (end 78.74 68.58) (width 1) (layer "F.Cu") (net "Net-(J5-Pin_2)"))
 (segment (start 93.98 49.53) (end 93.98 59.69) (width 1) (layer "F.Cu") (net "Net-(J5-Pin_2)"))
 (segment (start 83.82 66.04) (end 83.82 67.31) (width 1) (layer "F.Cu") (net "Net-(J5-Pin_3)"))
 (segment (start 83.82 67.31) (end 78.74 67.31) (width 1) (layer "F.Cu") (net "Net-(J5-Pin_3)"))
 (segment (start 91.44 58.42) (end 83.82 66.04) (width 1) (layer "F.Cu") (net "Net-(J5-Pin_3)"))
 (segment (start 91.44 49.53) (end 91.44 58.42) (width 1) (layer "F.Cu") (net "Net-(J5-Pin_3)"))
 (segment (start 96.52 60.96) (end 96.52 49.53) (width 1) (layer "F.Cu") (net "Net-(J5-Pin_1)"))
 (segment (start 78.74 69.85) (end 87.63 69.85) (width 1) (layer "F.Cu") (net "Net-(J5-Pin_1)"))
 (segment (start 87.63 69.85) (end 96.52 60.96) (width 1) (layer "F.Cu") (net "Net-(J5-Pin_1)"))
 (segment (start 103.58 43.18) (end 103.58 47.7) (width 1) (layer "F.Cu") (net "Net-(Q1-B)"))
 (segment (start 103.58 47.7) (end 105.41 49.53) (width 1) (layer "F.Cu") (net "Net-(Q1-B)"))
 (segment (start 90.45 43.18) (end 103.58 43.18) (width 1) (layer "F.Cu") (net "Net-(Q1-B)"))
 (segment (start 105.41 49.53) (end 106.68 49.53) (width 1) (layer "F.Cu") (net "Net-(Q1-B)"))
 (segment (start 116.84 43.18) (end 106.68 43.18) (width 1) (layer "F.Cu") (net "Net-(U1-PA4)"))
 (segment (start 120.65 46.99) (end 116.84 43.18) (width 1) (layer "F.Cu") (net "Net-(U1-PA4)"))
 (segment (start 72.815001 67.31) (end 71.12 65.614999) (width 1) (layer "F.Cu") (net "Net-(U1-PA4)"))
 (segment (start 71.12 58.42) (end 72.39 57.15) (width 1) (layer "F.Cu") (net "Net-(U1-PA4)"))
 (segment (start 72.815001 67.31) (end 72.602501 67.097499) (width 1) (layer "F.Cu") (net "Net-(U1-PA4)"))
 (segment (start 83.82 57.15) (end 88.9 57.15) (width 1) (layer "F.Cu") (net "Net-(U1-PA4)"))
 (segment (start 71.12 65.614999) (end 71.12 58.42) (width 1) (layer "F.Cu") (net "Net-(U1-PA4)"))
 (segment (start 99.06 57.15) (end 116.84 57.15) (width 1) (layer "F.Cu") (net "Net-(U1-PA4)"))
 (segment (start 73.79 67.31) (end 72.815001 67.31) (width 1) (layer "F.Cu") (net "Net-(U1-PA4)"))
 (segment (start 120.65 53.34) (end 120.65 46.99) (width 1) (layer "F.Cu") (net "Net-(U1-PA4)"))
 (segment (start 116.84 57.15) (end 120.65 53.34) (width 1) (layer "F.Cu") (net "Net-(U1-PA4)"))
 (via (at 72.39 57.15) (size 0.6) (drill 0.3) (layers "F.Cu" "B.Cu") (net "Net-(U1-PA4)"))
 (via (at 83.82 57.15) (size 0.6) (drill 0.3) (layers "F.Cu" "B.Cu") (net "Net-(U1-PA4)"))
 (via (at 99.06 57.15) (size 0.6) (drill 0.3) (layers "F.Cu" "B.Cu") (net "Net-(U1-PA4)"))
 (via (at 88.9 57.15) (size 0.6) (drill 0.3) (layers "F.Cu" "B.Cu") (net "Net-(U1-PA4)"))
 (via (at 99.06 57.15) (size 0.6) (drill 0.3) (layers "F.Cu" "B.Cu") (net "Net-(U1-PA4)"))
 (segment (start 72.39 57.15) (end 83.82 57.15) (width 1) (layer "B.Cu") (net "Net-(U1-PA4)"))
 (segment (start 88.9 57.15) (end 99.06 57.15) (width 1) (layer "B.Cu") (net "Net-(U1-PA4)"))
 (segment (start 71.12 71.12) (end 72.39 72.39) (width 1) (layer "F.Cu") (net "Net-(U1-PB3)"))
 (segment (start 60.325 71.12) (end 71.12 71.12) (width 1) (layer "F.Cu") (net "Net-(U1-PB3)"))
 (segment (start 51.435 62.23) (end 60.325 71.12) (width 1) (layer "F.Cu") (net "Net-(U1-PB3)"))
 (segment (start 72.39 72.39) (end 73.79 72.39) (width 1) (layer "F.Cu") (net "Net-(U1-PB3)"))
 (segment (start 46.355 73.66) (end 40.64 67.945) (width 1) (layer "F.Cu") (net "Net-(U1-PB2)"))
 (segment (start 64.77 40.64) (end 66.04 41.91) (width 1) (layer "F.Cu") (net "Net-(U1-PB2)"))
 (segment (start 66.04 58.42) (end 66.04 52.07) (width 1) (layer "F.Cu") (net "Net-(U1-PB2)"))
 (segment (start 74.36 73.66) (end 46.355 73.66) (width 1) (layer "F.Cu") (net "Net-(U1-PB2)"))
 (segment (start 40.64 67.945) (end 40.64 46.99) (width 1) (layer "F.Cu") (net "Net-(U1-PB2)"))
 (segment (start 46.99 40.64) (end 64.77 40.64) (width 1) (layer "F.Cu") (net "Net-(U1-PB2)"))
 (segment (start 59.055 62.23) (end 62.23 62.23) (width 1) (layer "F.Cu") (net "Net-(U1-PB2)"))
 (segment (start 62.23 62.23) (end 66.04 58.42) (width 1) (layer "F.Cu") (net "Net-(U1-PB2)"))
 (segment (start 40.64 46.99) (end 46.99 40.64) (width 1) (layer "F.Cu") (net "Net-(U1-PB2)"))
 (via (at 66.04 52.07) (size 0.6) (drill 0.3) (layers "F.Cu" "B.Cu") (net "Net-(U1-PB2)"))
 (via (at 66.04 41.91) (size 0.6) (drill 0.3) (layers "F.Cu" "B.Cu") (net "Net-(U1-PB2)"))
 (segment (start 66.04 41.91) (end 66.04 52.07) (width 1) (layer "B.Cu") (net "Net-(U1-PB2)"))
 (segment (start 64.135 69.85) (end 56.515 62.23) (width 1) (layer "F.Cu") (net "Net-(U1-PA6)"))
 (segment (start 73.79 69.85) (end 64.135 69.85) (width 1) (layer "F.Cu") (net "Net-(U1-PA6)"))
 (segment (start 53.975 62.23) (end 56.515 62.23) (width 1) (layer "F.Cu") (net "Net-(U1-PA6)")))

